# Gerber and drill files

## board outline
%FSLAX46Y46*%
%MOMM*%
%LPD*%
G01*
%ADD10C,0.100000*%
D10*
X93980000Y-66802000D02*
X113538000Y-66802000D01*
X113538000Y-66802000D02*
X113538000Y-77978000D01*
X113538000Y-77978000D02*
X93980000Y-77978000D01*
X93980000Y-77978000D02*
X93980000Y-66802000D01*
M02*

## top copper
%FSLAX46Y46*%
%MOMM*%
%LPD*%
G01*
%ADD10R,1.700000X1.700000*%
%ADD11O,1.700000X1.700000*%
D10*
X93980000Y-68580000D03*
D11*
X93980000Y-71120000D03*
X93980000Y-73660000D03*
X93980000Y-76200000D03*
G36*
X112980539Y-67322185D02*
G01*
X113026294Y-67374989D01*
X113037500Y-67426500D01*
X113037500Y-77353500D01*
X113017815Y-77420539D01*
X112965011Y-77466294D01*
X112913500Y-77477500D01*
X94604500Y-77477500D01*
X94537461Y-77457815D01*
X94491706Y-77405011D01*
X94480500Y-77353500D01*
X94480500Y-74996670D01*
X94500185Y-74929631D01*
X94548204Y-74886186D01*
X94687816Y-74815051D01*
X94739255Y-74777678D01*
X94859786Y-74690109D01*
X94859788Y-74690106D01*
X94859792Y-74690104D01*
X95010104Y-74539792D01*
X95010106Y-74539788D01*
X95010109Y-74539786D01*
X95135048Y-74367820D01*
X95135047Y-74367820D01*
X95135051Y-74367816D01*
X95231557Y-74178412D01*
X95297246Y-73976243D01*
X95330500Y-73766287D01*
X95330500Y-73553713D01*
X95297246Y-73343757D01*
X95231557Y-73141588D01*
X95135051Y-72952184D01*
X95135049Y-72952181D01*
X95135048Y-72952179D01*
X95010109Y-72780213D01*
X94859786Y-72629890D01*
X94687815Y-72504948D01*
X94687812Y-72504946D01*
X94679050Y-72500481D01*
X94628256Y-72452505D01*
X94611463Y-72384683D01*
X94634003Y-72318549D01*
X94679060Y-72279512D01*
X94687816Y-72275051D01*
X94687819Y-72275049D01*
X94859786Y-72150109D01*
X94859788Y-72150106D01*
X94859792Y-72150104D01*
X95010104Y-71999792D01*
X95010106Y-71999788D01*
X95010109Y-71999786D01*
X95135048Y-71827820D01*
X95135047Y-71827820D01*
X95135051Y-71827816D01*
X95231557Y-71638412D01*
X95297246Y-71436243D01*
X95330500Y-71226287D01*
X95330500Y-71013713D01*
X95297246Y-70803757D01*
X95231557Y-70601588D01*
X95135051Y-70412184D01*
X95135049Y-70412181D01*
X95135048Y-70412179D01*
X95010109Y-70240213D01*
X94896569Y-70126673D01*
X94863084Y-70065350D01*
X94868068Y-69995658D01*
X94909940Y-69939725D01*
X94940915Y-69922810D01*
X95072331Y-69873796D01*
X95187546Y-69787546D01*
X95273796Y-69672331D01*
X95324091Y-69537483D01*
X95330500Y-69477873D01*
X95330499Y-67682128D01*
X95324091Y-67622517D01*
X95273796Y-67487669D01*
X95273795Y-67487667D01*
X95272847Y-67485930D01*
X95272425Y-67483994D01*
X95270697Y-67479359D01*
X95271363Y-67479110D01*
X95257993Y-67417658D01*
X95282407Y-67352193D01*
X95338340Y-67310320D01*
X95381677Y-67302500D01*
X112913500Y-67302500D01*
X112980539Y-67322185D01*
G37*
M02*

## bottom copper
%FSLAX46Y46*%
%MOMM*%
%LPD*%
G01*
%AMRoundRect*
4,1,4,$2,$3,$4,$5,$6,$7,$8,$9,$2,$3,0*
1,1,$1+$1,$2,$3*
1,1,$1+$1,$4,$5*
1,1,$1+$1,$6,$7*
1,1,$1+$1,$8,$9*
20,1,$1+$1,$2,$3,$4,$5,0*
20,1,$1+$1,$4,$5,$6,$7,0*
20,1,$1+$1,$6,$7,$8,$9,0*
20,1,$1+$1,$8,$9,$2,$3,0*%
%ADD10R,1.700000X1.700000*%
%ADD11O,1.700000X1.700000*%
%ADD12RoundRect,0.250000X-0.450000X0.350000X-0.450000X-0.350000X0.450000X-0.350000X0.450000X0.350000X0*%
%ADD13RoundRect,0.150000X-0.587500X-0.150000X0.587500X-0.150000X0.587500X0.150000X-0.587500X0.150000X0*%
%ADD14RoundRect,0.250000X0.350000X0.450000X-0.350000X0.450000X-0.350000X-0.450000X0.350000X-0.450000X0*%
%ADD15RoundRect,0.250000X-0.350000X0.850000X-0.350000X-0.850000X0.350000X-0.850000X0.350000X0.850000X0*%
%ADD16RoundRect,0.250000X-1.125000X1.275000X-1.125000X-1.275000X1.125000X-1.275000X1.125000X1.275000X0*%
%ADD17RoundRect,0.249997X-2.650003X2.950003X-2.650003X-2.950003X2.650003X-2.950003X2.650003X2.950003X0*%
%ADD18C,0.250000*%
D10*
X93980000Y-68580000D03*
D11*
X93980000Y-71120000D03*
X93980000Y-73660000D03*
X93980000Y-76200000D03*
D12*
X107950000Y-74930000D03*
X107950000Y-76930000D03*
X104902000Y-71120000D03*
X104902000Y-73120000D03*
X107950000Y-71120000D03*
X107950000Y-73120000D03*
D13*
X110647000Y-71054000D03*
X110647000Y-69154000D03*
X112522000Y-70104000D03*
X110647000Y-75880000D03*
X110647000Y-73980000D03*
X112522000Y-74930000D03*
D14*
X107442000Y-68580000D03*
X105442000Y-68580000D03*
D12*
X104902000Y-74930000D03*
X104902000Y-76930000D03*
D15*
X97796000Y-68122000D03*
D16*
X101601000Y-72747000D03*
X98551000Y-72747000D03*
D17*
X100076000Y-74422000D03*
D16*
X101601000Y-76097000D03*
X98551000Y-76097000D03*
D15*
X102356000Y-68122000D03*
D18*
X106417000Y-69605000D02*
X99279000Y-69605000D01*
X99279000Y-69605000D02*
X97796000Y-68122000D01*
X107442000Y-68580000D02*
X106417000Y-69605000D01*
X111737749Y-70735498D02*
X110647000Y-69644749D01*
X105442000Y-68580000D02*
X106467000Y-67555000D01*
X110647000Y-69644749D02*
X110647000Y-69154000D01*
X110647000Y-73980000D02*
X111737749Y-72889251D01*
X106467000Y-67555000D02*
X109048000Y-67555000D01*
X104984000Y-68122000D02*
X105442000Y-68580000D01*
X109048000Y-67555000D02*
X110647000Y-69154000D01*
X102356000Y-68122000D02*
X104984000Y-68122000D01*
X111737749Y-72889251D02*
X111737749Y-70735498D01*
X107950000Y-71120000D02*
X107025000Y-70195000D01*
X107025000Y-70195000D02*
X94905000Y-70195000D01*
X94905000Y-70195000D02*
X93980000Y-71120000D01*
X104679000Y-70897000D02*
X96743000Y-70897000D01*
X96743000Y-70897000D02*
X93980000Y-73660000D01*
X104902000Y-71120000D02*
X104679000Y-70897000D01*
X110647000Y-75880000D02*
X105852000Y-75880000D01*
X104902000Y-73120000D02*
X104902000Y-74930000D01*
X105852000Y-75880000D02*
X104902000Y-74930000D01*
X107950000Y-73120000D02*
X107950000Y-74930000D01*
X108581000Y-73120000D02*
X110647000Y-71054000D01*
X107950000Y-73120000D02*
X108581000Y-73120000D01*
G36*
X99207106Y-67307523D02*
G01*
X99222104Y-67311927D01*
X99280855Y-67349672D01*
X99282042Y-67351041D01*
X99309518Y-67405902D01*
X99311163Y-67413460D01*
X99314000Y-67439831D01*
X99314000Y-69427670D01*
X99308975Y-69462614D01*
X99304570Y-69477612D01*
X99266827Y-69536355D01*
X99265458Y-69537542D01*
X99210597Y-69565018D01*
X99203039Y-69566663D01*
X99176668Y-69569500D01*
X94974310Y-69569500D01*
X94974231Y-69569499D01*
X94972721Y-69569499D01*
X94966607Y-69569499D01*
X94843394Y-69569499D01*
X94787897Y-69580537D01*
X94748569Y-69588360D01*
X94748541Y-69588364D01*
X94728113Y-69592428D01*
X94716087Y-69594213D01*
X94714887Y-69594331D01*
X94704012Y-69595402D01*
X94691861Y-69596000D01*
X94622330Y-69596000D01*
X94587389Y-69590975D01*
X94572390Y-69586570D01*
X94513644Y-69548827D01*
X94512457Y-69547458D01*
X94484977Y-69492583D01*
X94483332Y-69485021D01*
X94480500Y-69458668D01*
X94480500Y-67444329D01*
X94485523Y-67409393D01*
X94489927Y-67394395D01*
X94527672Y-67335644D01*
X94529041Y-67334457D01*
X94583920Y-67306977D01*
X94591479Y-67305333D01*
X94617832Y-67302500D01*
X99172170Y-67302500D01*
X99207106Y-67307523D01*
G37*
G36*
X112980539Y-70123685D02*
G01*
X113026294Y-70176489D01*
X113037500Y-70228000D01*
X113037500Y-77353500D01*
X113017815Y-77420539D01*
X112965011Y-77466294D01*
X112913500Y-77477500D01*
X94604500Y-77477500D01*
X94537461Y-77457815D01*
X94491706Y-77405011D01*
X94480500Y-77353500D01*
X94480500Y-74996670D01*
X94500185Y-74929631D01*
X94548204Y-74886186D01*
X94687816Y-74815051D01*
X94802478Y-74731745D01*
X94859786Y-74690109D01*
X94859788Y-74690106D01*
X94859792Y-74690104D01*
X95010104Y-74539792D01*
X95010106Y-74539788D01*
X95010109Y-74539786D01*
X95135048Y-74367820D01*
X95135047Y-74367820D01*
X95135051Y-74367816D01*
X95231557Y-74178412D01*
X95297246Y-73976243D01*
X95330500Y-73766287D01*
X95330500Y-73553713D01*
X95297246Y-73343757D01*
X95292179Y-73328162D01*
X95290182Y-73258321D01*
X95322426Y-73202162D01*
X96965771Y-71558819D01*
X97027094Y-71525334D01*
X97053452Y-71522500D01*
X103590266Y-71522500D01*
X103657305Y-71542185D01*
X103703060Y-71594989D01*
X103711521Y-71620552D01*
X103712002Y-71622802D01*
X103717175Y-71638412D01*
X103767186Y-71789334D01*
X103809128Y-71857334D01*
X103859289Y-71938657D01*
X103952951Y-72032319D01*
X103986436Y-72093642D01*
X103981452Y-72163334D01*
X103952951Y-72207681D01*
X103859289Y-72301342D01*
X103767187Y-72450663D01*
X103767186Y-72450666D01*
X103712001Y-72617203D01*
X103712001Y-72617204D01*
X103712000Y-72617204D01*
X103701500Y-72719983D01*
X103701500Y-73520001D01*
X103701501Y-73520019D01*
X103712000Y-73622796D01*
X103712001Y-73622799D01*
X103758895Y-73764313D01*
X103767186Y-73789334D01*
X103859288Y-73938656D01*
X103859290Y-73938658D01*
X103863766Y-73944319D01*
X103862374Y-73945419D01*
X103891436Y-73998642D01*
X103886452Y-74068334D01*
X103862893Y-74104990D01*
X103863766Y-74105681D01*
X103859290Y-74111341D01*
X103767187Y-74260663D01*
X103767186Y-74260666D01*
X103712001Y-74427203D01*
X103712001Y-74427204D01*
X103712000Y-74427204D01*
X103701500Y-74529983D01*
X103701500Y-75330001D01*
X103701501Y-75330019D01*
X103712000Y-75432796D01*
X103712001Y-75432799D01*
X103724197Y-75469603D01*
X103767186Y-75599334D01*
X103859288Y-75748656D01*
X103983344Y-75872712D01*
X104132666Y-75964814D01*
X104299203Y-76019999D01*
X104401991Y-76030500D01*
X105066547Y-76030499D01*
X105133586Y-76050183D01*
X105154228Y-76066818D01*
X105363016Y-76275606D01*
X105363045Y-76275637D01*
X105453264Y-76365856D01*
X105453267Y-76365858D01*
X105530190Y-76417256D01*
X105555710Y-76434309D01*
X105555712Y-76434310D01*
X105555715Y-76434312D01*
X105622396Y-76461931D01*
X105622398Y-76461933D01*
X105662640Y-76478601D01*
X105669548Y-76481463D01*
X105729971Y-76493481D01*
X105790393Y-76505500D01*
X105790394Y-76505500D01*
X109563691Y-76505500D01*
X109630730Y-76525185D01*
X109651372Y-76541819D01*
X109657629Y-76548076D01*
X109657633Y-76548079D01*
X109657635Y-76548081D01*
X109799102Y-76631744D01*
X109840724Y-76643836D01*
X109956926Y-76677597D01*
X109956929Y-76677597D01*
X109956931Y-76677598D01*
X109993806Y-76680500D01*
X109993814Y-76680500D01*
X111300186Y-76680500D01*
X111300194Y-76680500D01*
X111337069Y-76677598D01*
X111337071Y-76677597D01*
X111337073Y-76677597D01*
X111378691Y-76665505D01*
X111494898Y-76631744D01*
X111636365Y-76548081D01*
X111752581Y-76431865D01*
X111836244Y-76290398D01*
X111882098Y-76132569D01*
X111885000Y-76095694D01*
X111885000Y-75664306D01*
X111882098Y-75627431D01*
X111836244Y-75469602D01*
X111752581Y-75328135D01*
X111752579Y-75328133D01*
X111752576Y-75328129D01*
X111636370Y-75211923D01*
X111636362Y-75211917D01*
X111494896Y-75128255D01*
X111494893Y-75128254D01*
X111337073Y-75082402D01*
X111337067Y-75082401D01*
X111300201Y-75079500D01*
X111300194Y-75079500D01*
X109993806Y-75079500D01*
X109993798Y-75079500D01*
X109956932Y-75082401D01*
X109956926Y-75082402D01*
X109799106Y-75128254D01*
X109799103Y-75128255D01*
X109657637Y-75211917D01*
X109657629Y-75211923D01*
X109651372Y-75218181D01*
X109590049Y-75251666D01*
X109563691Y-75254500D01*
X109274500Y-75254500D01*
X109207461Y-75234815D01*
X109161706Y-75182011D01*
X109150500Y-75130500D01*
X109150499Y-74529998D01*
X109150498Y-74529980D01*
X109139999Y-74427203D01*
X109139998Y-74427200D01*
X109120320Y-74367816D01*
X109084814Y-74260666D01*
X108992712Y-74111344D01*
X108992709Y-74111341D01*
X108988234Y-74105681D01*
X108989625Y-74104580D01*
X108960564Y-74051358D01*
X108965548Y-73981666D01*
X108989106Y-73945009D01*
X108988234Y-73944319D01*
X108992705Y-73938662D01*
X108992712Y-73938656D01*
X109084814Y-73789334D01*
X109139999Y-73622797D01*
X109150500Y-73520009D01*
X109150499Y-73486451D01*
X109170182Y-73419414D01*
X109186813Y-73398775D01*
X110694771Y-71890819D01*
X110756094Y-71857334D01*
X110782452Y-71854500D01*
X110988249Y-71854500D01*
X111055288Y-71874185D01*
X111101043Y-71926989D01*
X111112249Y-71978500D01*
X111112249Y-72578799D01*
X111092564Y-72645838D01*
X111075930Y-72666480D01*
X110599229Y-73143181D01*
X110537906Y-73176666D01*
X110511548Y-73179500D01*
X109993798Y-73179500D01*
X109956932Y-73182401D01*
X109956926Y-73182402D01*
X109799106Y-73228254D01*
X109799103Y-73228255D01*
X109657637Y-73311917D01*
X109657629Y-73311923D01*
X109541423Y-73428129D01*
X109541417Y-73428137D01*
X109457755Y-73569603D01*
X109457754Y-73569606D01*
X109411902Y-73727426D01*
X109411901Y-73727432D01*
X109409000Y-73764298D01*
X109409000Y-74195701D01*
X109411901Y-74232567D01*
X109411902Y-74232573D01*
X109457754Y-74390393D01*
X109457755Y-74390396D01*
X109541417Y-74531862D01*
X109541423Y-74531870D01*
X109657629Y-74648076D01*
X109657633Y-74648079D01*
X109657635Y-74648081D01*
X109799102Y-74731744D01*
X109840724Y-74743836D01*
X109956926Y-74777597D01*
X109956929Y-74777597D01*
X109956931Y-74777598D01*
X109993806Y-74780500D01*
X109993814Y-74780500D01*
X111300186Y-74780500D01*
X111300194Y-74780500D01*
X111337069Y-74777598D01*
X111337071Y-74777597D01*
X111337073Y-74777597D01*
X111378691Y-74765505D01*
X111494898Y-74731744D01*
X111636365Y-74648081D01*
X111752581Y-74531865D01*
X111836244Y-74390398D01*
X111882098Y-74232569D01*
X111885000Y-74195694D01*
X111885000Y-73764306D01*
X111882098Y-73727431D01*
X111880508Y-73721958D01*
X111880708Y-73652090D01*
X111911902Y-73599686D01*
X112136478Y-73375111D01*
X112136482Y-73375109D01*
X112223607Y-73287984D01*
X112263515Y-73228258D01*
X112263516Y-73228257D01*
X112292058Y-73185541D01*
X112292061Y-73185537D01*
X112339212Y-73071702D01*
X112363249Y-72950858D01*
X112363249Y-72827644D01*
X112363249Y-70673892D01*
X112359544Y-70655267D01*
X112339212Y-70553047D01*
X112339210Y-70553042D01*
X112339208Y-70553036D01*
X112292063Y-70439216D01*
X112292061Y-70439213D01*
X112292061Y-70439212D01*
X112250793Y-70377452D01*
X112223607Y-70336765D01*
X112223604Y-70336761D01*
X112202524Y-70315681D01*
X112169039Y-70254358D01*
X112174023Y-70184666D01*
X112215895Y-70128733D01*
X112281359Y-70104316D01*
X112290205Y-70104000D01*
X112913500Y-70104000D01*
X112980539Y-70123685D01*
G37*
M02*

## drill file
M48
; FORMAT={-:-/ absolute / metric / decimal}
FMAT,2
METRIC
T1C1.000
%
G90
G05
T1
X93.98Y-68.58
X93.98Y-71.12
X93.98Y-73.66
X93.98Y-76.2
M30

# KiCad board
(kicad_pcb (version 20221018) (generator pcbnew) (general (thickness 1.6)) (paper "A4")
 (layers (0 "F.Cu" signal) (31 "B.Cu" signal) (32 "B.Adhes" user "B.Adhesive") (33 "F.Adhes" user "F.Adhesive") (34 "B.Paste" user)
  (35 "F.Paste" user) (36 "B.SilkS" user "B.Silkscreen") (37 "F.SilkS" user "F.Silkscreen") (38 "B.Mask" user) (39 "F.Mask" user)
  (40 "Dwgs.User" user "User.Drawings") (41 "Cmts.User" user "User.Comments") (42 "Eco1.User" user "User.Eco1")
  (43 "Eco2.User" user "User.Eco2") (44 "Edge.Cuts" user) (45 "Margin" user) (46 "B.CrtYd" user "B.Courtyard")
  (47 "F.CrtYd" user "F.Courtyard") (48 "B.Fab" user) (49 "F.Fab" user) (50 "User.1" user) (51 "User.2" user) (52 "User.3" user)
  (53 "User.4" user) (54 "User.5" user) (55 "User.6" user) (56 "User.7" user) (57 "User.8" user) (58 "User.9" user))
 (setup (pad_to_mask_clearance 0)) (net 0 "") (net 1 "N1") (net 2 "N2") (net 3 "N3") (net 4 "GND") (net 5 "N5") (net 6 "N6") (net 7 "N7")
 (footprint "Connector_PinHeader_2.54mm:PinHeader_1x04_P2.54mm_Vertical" (layer "F.Cu") (at 93.98 68.58)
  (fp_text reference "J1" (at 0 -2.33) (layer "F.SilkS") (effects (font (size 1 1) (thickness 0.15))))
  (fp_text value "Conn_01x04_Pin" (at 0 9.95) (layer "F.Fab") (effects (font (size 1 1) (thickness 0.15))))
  (pad "1" thru_hole rect (at 0 0) (size 1.7 1.7) (drill 1) (layers "*.Cu" "*.Mask") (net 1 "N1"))
  (pad "2" thru_hole oval (at 0 2.54) (size 1.7 1.7) (drill 1) (layers "*.Cu" "*.Mask") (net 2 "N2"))
  (pad "3" thru_hole oval (at 0 5.08) (size 1.7 1.7) (drill 1) (layers "*.Cu" "*.Mask") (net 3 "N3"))
  (pad "4" thru_hole oval (at 0 7.62) (size 1.7 1.7) (drill 1) (layers "*.Cu" "*.Mask") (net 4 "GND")))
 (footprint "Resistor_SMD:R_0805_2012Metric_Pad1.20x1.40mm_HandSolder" (layer "B.Cu") (at 107.95 75.93 -90)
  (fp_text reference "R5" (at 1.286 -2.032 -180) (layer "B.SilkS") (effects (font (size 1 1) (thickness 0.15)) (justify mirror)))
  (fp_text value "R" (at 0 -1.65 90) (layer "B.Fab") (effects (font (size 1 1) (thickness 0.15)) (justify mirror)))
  (pad "1" smd roundrect (at -1 0 270) (size 1.2 1.4) (layers "B.Cu" "B.Paste" "B.Mask") (roundrect_rratio 0.2083333333) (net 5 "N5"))
  (pad "2" smd roundrect (at 1 0 270) (size 1.2 1.4) (layers "B.Cu" "B.Paste" "B.Mask") (roundrect_rratio 0.2083333333) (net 4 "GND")))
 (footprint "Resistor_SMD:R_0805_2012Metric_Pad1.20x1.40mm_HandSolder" (layer "B.Cu") (at 104.902 72.12 -90)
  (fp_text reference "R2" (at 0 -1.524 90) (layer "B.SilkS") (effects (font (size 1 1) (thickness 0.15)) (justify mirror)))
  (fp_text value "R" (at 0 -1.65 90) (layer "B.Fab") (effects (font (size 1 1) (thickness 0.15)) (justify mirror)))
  (pad "1" smd roundrect (at -1 0 270) (size 1.2 1.4) (layers "B.Cu" "B.Paste" "B.Mask") (roundrect_rratio 0.2083333333) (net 3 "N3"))
  (pad "2" smd roundrect (at 1 0 270) (size 1.2 1.4) (layers "B.Cu" "B.Paste" "B.Mask") (roundrect_rratio 0.2083333333) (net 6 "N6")))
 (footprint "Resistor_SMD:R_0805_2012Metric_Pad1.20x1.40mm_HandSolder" (layer "B.Cu") (at 107.95 72.12 -90)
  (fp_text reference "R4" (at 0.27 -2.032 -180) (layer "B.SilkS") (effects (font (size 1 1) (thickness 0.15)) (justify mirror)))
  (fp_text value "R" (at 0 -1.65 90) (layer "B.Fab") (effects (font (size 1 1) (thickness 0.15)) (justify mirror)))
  (pad "1" smd roundrect (at -1 0 270) (size 1.2 1.4) (layers "B.Cu" "B.Paste" "B.Mask") (roundrect_rratio 0.2083333333) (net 2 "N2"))
  (pad "2" smd roundrect (at 1 0 270) (size 1.2 1.4) (layers "B.Cu" "B.Paste" "B.Mask") (roundrect_rratio 0.2083333333) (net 5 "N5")))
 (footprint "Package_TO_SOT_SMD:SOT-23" (layer "B.Cu") (at 111.5845 70.104)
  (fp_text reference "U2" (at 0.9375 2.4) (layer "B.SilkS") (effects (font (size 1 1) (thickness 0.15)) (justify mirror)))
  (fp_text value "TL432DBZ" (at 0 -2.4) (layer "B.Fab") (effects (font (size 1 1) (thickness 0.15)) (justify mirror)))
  (pad "1" smd roundrect (at -0.9375 0.95) (size 1.475 0.6) (layers "B.Cu" "B.Paste" "B.Mask") (roundrect_rratio 0.25) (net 5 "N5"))
  (pad "2" smd roundrect (at -0.9375 -0.95) (size 1.475 0.6) (layers "B.Cu" "B.Paste" "B.Mask") (roundrect_rratio 0.25) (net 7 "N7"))
  (pad "3" smd roundrect (at 0.9375 0) (size 1.475 0.6) (layers "B.Cu" "B.Paste" "B.Mask") (roundrect_rratio 0.25) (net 4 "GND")))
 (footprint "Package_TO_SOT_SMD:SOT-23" (layer "B.Cu") (at 111.5845 74.93)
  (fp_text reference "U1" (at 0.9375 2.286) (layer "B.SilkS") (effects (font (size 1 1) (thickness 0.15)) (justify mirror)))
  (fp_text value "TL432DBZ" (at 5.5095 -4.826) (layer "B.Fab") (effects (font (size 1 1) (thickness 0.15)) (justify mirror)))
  (pad "1" smd roundrect (at -0.9375 0.95) (size 1.475 0.6) (layers "B.Cu" "B.Paste" "B.Mask") (roundrect_rratio 0.25) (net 6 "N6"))
  (pad "2" smd roundrect (at -0.9375 -0.95) (size 1.475 0.6) (layers "B.Cu" "B.Paste" "B.Mask") (roundrect_rratio 0.25) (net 7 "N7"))
  (pad "3" smd roundrect (at 0.9375 0) (size 1.475 0.6) (layers "B.Cu" "B.Paste" "B.Mask") (roundrect_rratio 0.25) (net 4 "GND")))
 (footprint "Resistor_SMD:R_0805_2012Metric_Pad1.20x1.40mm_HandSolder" (layer "B.Cu") (at 106.442 68.58 180)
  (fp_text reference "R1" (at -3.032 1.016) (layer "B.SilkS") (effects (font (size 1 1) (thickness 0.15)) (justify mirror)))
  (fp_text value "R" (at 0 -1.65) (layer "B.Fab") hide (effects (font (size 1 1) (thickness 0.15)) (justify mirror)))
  (pad "1" smd roundrect (at -1 0 180) (size 1.2 1.4) (layers "B.Cu" "B.Paste" "B.Mask") (roundrect_rratio 0.2083333333) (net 1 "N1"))
  (pad "2" smd roundrect (at 1 0 180) (size 1.2 1.4) (layers "B.Cu" "B.Paste" "B.Mask") (roundrect_rratio 0.2083333333) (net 7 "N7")))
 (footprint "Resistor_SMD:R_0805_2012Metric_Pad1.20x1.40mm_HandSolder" (layer "B.Cu") (at 104.902 75.93 -90)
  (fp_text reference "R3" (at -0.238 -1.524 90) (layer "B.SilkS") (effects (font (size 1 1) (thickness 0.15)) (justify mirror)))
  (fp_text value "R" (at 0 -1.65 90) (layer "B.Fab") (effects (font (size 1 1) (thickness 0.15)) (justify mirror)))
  (pad "1" smd roundrect (at -1 0 270) (size 1.2 1.4) (layers "B.Cu" "B.Paste" "B.Mask") (roundrect_rratio 0.2083333333) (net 6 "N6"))
  (pad "2" smd roundrect (at 1 0 270) (size 1.2 1.4) (layers "B.Cu" "B.Paste" "B.Mask") (roundrect_rratio 0.2083333333) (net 4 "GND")))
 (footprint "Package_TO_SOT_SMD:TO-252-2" (layer "B.Cu") (at 100.076 73.162 -90)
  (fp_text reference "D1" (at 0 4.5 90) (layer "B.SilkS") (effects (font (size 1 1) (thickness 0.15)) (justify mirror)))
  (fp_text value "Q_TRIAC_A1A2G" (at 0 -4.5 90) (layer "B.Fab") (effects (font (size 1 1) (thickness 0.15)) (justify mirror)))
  (pad "1" smd roundrect (at -5.04 2.28 270) (size 2.2 1.2) (layers "B.Cu" "B.Paste" "B.Mask") (roundrect_rratio 0.2083333333) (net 1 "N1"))
  (pad "2" smd roundrect (at -0.415 -1.525 270) (size 3.05 2.75) (layers "B.Cu" "B.Paste") (roundrect_rratio 0.09090909091) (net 4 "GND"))
  (pad "2" smd roundrect (at -0.415 1.525 270) (size 3.05 2.75) (layers "B.Cu" "B.Paste") (roundrect_rratio 0.09090909091) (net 4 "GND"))
  (pad "2" smd roundrect (at 1.26 0 270) (size 6.4 5.8) (layers "B.Cu" "B.Mask") (roundrect_rratio 0.04310293103) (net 4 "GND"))
  (pad "2" smd roundrect (at 2.935 -1.525 270) (size 3.05 2.75) (layers "B.Cu" "B.Paste") (roundrect_rratio 0.09090909091) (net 4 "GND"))
  (pad "2" smd roundrect (at 2.935 1.525 270) (size 3.05 2.75) (layers "B.Cu" "B.Paste") (roundrect_rratio 0.09090909091) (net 4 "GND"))
  (pad "3" smd roundrect (at -5.04 -2.28 270) (size 2.2 1.2) (layers "B.Cu" "B.Paste" "B.Mask") (roundrect_rratio 0.2083333333) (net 7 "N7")))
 (gr_line (start 93.98 66.802) (end 113.538 66.802) (stroke (width 0.1) (type default)) (layer "Edge.Cuts"))
 (gr_line (start 113.538 66.802) (end 113.538 77.978) (stroke (width 0.1) (type default)) (layer "Edge.Cuts"))
 (gr_line (start 113.538 77.978) (end 93.98 77.978) (stroke (width 0.1) (type default)) (layer "Edge.Cuts"))
 (gr_line (start 93.98 77.978) (end 93.98 66.802) (stroke (width 0.1) (type default)) (layer "Edge.Cuts"))
 (segment (start 106.417 69.605) (end 99.279 69.605) (width 0.25) (layer "B.Cu") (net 1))
 (segment (start 99.279 69.605) (end 97.796 68.122) (width 0.25) (layer "B.Cu") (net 1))
 (segment (start 107.442 68.58) (end 106.417 69.605) (width 0.25) (layer "B.Cu") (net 1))
 (segment (start 111.737749 70.735498) (end 110.647 69.644749) (width 0.25) (layer "B.Cu") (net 7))
 (segment (start 105.442 68.58) (end 106.467 67.555) (width 0.25) (layer "B.Cu") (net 7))
 (segment (start 110.647 69.644749) (end 110.647 69.154) (width 0.25) (layer "B.Cu") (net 7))
 (segment (start 110.647 73.98) (end 111.737749 72.889251) (width 0.25) (layer "B.Cu") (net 7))
 (segment (start 106.467 67.555) (end 109.048 67.555) (width 0.25) (layer "B.Cu") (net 7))
 (segment (start 104.984 68.122) (end 105.442 68.58) (width 0.25) (layer "B.Cu") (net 7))
 (segment (start 109.048 67.555) (end 110.647 69.154) (width 0.25) (layer "B.Cu") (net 7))
 (segment (start 102.356 68.122) (end 104.984 68.122) (width 0.25) (layer "B.Cu") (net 7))
 (segment (start 111.737749 72.889251) (end 111.737749 70.735498) (width 0.25) (layer "B.Cu") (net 7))
 (segment (start 107.95 71.12) (end 107.025 70.195) (width 0.25) (layer "B.Cu") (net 2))
 (segment (start 107.025 70.195) (end 94.905 70.195) (width 0.25) (layer "B.Cu") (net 2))
 (segment (start 94.905 70.195) (end 93.98 71.12) (width 0.25) (layer "B.Cu") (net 2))
 (segment (start 104.679 70.897) (end 96.743 70.897) (width 0.25) (layer "B.Cu") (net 3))
 (segment (start 96.743 70.897) (end 93.98 73.66) (width 0.25) (layer "B.Cu") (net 3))
 (segment (start 104.902 71.12) (end 104.679 70.897) (width 0.25) (layer "B.Cu") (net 3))
 (segment (start 110.647 75.88) (end 105.852 75.88) (width 0.25) (layer "B.Cu") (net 6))
 (segment (start 104.902 73.12) (end 104.902 74.93) (width 0.25) (layer "B.Cu") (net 6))
 (segment (start 105.852 75.88) (end 104.902 74.93) (width 0.25) (layer "B.Cu") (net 6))
 (segment (start 107.95 73.12) (end 107.95 74.93) (width 0.25) (layer "B.Cu") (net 5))
 (segment (start 108.581 73.12) (end 110.647 71.054) (width 0.25) (layer "B.Cu") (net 5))
 (segment (start 107.95 73.12) (end 108.581 73.12) (width 0.25) (layer "B.Cu") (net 5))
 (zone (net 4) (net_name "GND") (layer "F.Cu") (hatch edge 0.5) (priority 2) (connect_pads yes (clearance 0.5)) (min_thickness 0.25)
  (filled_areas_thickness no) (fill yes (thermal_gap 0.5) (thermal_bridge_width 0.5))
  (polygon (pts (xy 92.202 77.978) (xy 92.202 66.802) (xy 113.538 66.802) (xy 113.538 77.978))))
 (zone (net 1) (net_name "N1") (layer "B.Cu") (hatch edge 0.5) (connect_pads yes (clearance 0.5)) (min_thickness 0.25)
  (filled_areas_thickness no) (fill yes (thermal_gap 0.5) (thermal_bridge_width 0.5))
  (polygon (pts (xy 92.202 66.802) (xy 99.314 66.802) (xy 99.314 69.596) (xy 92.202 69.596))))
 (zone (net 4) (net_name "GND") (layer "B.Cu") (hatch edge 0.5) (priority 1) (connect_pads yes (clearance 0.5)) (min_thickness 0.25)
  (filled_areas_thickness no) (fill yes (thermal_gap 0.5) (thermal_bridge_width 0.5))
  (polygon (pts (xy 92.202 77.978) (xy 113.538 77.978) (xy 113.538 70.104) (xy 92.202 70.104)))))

